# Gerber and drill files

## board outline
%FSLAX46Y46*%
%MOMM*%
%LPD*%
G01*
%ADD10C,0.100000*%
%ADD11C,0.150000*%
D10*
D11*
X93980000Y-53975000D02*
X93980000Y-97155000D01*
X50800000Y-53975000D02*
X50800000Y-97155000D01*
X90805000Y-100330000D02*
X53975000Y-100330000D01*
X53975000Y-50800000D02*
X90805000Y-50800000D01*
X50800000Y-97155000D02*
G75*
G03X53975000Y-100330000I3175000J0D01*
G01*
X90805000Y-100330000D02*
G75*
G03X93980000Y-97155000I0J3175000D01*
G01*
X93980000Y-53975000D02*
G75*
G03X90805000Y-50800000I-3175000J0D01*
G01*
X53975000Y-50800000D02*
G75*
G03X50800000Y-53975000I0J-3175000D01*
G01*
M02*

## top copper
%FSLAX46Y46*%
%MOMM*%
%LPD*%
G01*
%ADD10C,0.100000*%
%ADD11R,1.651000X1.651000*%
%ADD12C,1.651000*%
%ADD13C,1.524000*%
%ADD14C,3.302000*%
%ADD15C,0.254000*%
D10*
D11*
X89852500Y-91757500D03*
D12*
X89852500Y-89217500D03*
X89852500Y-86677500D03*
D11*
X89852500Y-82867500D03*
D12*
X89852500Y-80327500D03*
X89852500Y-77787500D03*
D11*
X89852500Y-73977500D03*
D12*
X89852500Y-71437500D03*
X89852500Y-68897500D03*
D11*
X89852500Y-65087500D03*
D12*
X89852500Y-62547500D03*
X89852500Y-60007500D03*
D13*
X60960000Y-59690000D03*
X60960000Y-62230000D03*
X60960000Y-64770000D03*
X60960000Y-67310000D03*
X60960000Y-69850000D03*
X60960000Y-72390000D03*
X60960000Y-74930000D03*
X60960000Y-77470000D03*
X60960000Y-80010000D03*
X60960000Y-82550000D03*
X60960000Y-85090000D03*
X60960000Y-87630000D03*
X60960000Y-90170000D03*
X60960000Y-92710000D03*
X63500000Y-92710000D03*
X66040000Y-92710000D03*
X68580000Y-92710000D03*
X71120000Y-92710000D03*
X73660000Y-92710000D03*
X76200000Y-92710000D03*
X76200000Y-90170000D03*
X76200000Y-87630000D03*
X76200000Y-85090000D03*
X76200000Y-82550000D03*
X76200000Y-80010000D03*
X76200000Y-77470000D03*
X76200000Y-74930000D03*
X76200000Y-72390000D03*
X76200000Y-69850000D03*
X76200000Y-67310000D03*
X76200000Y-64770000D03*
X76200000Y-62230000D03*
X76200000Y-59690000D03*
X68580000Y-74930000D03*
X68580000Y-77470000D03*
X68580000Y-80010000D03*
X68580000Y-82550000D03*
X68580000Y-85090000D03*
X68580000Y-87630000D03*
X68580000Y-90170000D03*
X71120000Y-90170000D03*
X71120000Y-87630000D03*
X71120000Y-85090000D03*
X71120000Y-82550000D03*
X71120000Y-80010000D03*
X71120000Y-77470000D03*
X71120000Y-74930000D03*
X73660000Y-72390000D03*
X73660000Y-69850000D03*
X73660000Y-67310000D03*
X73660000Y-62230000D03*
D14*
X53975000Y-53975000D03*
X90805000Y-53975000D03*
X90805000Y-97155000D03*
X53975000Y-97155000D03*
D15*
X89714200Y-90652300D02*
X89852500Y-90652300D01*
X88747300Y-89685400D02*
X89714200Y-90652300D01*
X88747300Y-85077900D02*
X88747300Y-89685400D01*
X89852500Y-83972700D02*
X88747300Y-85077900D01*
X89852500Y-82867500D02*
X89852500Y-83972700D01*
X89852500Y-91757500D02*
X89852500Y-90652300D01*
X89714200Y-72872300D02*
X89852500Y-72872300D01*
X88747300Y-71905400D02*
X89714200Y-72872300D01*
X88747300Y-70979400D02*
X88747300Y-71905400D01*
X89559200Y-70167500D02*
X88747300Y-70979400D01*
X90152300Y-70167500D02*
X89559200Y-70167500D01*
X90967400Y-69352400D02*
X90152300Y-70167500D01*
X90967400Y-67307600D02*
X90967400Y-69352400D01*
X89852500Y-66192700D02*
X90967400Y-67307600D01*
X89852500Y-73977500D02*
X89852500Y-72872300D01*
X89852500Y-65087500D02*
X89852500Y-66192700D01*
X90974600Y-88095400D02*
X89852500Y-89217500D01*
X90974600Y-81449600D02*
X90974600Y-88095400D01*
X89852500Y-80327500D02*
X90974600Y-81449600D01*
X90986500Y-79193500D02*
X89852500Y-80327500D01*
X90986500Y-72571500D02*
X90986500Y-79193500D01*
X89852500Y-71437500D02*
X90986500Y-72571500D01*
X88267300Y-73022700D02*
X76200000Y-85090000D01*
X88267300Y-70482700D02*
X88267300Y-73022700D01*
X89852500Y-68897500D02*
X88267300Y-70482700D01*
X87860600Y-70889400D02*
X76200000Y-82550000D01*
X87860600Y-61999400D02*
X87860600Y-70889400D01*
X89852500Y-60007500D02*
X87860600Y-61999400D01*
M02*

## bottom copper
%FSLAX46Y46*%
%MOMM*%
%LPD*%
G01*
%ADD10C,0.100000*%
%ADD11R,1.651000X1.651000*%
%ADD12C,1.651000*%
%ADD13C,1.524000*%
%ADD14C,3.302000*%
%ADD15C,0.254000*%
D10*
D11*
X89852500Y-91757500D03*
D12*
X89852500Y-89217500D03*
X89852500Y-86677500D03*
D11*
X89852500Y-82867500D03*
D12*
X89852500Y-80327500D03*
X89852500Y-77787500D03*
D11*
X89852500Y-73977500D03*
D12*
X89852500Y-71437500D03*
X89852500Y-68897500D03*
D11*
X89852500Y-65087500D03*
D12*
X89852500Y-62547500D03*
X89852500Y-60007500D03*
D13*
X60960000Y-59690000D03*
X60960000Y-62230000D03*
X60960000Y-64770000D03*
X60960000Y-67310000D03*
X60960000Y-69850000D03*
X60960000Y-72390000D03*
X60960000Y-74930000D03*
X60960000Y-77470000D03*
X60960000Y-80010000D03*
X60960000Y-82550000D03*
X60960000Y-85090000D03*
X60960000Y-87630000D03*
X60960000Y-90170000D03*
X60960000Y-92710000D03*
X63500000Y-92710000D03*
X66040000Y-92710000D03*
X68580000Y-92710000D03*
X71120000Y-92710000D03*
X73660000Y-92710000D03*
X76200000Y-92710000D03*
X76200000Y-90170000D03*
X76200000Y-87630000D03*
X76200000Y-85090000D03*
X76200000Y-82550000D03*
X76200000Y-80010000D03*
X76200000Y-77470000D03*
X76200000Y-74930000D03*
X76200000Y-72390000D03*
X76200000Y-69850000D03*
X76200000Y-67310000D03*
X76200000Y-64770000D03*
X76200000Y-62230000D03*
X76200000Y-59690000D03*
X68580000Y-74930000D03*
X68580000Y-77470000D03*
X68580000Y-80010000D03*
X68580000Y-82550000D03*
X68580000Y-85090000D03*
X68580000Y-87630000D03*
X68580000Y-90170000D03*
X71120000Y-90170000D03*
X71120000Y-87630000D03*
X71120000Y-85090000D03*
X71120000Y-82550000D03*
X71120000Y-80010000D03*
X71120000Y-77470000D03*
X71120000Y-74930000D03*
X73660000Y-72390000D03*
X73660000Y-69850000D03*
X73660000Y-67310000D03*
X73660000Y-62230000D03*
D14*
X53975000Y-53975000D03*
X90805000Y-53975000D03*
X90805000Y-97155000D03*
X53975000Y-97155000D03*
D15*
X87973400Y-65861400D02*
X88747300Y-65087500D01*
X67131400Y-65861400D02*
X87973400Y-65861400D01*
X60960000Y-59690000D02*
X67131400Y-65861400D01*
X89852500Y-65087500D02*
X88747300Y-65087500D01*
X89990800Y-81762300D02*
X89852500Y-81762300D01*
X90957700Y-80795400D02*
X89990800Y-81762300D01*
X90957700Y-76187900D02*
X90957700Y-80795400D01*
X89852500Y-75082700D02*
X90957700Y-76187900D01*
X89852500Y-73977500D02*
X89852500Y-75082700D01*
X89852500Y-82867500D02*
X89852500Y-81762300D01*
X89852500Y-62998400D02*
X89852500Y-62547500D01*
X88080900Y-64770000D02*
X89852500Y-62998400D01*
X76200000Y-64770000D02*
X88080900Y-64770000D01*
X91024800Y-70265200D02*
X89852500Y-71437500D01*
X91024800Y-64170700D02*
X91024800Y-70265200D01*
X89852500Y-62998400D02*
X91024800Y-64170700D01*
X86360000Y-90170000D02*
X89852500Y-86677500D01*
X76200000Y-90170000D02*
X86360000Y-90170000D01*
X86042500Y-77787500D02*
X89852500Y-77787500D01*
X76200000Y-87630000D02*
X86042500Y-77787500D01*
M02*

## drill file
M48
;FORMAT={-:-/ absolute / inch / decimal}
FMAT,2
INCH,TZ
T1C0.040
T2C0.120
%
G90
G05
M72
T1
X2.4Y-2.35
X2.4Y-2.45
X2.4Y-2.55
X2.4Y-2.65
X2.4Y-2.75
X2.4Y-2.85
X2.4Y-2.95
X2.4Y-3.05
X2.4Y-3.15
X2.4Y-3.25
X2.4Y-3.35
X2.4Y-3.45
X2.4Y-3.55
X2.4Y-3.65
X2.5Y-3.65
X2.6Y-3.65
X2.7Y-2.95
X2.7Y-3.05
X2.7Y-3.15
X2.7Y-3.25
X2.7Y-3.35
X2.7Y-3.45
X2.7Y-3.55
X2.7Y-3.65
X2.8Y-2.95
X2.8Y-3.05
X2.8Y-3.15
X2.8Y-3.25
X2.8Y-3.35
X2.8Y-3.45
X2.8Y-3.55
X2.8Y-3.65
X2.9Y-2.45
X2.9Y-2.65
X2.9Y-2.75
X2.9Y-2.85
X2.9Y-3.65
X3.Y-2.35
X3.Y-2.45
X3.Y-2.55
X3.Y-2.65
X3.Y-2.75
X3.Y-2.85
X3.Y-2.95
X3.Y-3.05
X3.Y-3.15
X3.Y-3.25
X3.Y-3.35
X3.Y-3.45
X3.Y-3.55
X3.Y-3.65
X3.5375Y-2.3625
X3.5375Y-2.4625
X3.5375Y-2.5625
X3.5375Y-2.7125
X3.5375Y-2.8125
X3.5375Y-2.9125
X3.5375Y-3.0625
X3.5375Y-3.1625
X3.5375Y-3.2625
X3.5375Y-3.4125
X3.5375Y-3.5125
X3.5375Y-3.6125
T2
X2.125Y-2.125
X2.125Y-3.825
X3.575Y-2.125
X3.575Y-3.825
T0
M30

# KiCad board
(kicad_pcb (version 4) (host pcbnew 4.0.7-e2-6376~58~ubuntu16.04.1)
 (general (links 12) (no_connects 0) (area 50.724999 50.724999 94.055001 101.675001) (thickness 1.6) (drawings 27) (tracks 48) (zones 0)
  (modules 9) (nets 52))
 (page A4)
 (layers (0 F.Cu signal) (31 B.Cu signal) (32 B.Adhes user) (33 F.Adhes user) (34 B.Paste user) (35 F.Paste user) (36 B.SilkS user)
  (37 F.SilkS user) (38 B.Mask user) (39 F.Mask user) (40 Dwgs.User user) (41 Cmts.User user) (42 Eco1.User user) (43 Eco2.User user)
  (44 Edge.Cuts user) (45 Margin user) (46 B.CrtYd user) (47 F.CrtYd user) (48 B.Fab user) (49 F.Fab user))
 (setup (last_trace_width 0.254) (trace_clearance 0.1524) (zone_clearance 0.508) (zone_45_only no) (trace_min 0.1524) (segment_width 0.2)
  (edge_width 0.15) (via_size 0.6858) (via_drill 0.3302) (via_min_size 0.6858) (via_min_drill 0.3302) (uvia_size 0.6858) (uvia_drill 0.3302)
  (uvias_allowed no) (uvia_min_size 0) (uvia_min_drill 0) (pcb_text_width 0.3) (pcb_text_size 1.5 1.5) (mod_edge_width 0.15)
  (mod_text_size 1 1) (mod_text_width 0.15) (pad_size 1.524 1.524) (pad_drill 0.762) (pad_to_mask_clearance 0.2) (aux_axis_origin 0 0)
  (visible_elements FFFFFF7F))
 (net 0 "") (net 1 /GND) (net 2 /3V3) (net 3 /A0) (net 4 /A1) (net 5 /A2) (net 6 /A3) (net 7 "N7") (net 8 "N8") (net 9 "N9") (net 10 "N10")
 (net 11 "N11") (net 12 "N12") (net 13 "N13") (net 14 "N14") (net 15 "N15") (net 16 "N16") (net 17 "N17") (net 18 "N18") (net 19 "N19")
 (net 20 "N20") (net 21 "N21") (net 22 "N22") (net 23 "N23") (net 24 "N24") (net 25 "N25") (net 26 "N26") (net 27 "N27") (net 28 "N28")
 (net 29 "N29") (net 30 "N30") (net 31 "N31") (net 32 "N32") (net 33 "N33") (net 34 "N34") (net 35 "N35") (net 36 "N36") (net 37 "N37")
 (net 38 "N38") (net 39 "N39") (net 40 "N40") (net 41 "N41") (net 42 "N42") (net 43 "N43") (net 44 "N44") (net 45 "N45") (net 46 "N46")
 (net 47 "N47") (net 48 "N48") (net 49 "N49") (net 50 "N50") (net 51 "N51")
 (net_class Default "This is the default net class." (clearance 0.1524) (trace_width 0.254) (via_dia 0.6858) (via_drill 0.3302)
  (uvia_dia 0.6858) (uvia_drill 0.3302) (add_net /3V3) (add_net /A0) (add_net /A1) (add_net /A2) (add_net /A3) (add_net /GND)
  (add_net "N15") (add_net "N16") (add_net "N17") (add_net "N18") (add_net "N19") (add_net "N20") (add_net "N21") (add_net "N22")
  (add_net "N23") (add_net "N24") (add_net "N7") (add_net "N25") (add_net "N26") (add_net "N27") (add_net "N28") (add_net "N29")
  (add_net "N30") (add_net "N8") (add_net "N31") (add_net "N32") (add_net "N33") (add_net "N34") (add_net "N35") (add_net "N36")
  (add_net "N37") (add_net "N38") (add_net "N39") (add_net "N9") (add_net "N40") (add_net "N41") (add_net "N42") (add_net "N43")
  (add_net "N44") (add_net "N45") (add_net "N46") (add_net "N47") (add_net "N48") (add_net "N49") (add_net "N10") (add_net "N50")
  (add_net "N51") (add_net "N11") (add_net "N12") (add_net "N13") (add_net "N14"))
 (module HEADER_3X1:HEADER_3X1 (layer F.Cu) (at 89.8525 89.2175 90)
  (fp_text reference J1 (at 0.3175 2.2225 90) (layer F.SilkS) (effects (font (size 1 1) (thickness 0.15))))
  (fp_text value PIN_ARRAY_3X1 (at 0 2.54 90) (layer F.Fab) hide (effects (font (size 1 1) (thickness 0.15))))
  (pad 1 thru_hole rect (at -2.54 0 90) (size 1.651 1.651) (drill 1.016) (layers *.Cu *.Mask) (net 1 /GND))
  (pad 2 thru_hole circle (at 0 0 90) (size 1.651 1.651) (drill 1.016) (layers *.Cu *.Mask) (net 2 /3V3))
  (pad 3 thru_hole circle (at 2.54 0 90) (size 1.651 1.651) (drill 1.016) (layers *.Cu *.Mask) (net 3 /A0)))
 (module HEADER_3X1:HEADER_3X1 (layer F.Cu) (at 89.8525 80.3275 90)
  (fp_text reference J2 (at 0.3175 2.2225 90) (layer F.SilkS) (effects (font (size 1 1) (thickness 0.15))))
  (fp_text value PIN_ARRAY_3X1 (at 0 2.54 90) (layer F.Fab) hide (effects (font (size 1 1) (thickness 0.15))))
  (pad 1 thru_hole rect (at -2.54 0 90) (size 1.651 1.651) (drill 1.016) (layers *.Cu *.Mask) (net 1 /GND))
  (pad 2 thru_hole circle (at 0 0 90) (size 1.651 1.651) (drill 1.016) (layers *.Cu *.Mask) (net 2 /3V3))
  (pad 3 thru_hole circle (at 2.54 0 90) (size 1.651 1.651) (drill 1.016) (layers *.Cu *.Mask) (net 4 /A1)))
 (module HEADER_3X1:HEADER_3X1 (layer F.Cu) (at 89.8525 71.4375 90)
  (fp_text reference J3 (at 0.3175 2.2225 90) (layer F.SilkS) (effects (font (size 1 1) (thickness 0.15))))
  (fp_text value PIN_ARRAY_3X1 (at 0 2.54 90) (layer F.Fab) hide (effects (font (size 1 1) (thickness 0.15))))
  (pad 1 thru_hole rect (at -2.54 0 90) (size 1.651 1.651) (drill 1.016) (layers *.Cu *.Mask) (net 1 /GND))
  (pad 2 thru_hole circle (at 0 0 90) (size 1.651 1.651) (drill 1.016) (layers *.Cu *.Mask) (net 2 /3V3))
  (pad 3 thru_hole circle (at 2.54 0 90) (size 1.651 1.651) (drill 1.016) (layers *.Cu *.Mask) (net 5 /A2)))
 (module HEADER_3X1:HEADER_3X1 (layer F.Cu) (at 89.8525 62.5475 90)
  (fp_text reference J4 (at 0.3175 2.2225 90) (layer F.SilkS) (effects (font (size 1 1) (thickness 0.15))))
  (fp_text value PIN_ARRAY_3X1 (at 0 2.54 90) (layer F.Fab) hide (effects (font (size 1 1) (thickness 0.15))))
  (pad 1 thru_hole rect (at -2.54 0 90) (size 1.651 1.651) (drill 1.016) (layers *.Cu *.Mask) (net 1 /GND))
  (pad 2 thru_hole circle (at 0 0 90) (size 1.651 1.651) (drill 1.016) (layers *.Cu *.Mask) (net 2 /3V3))
  (pad 3 thru_hole circle (at 2.54 0 90) (size 1.651 1.651) (drill 1.016) (layers *.Cu *.Mask) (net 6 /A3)))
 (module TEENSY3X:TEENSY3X (layer F.Cu) (at 68.58 76.2)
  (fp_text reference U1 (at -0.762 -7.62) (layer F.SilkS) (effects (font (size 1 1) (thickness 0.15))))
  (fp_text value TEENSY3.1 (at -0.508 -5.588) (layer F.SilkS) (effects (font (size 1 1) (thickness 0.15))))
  (pad 1 thru_hole circle (at -7.62 -16.51) (size 1.524 1.524) (drill 1.016) (layers *.Cu *.Mask F.SilkS) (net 1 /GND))
  (pad 2 thru_hole circle (at -7.62 -13.97) (size 1.524 1.524) (drill 1.016) (layers *.Cu *.Mask F.SilkS) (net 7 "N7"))
  (pad 3 thru_hole circle (at -7.62 -11.43) (size 1.524 1.524) (drill 1.016) (layers *.Cu *.Mask F.SilkS) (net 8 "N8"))
  (pad 4 thru_hole circle (at -7.62 -8.89) (size 1.524 1.524) (drill 1.016) (layers *.Cu *.Mask F.SilkS) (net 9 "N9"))
  (pad 5 thru_hole circle (at -7.62 -6.35) (size 1.524 1.524) (drill 1.016) (layers *.Cu *.Mask F.SilkS) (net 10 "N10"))
  (pad 6 thru_hole circle (at -7.62 -3.81) (size 1.524 1.524) (drill 1.016) (layers *.Cu *.Mask F.SilkS) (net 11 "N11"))
  (pad 7 thru_hole circle (at -7.62 -1.27) (size 1.524 1.524) (drill 1.016) (layers *.Cu *.Mask F.SilkS) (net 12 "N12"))
  (pad 8 thru_hole circle (at -7.62 1.27) (size 1.524 1.524) (drill 1.016) (layers *.Cu *.Mask F.SilkS) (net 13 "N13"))
  (pad 9 thru_hole circle (at -7.62 3.81) (size 1.524 1.524) (drill 1.016) (layers *.Cu *.Mask F.SilkS) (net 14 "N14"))
  (pad 10 thru_hole circle (at -7.62 6.35) (size 1.524 1.524) (drill 1.016) (layers *.Cu *.Mask F.SilkS) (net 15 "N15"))
  (pad 11 thru_hole circle (at -7.62 8.89) (size 1.524 1.524) (drill 1.016) (layers *.Cu *.Mask F.SilkS) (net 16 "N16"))
  (pad 12 thru_hole circle (at -7.62 11.43) (size 1.524 1.524) (drill 1.016) (layers *.Cu *.Mask F.SilkS) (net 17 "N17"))
  (pad 13 thru_hole circle (at -7.62 13.97) (size 1.524 1.524) (drill 1.016) (layers *.Cu *.Mask F.SilkS) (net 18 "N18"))
  (pad 14 thru_hole circle (at -7.62 16.51) (size 1.524 1.524) (drill 1.016) (layers *.Cu *.Mask F.SilkS) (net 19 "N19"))
  (pad 15 thru_hole circle (at -5.08 16.51) (size 1.524 1.524) (drill 1.016) (layers *.Cu *.Mask F.SilkS) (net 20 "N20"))
  (pad 16 thru_hole circle (at -2.54 16.51) (size 1.524 1.524) (drill 1.016) (layers *.Cu *.Mask F.SilkS) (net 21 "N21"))
  (pad 17 thru_hole circle (at 0 16.51) (size 1.524 1.524) (drill 1.016) (layers *.Cu *.Mask F.SilkS) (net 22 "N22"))
  (pad 18 thru_hole circle (at 2.54 16.51) (size 1.524 1.524) (drill 1.016) (layers *.Cu *.Mask F.SilkS) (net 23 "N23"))
  (pad 19 thru_hole circle (at 5.08 16.51) (size 1.524 1.524) (drill 1.016) (layers *.Cu *.Mask F.SilkS) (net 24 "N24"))
  (pad 20 thru_hole circle (at 7.62 16.51) (size 1.524 1.524) (drill 1.016) (layers *.Cu *.Mask F.SilkS) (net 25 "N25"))
  (pad 21 thru_hole circle (at 7.62 13.97) (size 1.524 1.524) (drill 1.016) (layers *.Cu *.Mask F.SilkS) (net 3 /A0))
  (pad 22 thru_hole circle (at 7.62 11.43) (size 1.524 1.524) (drill 1.016) (layers *.Cu *.Mask F.SilkS) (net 4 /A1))
  (pad 23 thru_hole circle (at 7.62 8.89) (size 1.524 1.524) (drill 1.016) (layers *.Cu *.Mask F.SilkS) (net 5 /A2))
  (pad 24 thru_hole circle (at 7.62 6.35) (size 1.524 1.524) (drill 1.016) (layers *.Cu *.Mask F.SilkS) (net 6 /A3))
  (pad 25 thru_hole circle (at 7.62 3.81) (size 1.524 1.524) (drill 1.016) (layers *.Cu *.Mask F.SilkS) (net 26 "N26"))
  (pad 26 thru_hole circle (at 7.62 1.27) (size 1.524 1.524) (drill 1.016) (layers *.Cu *.Mask F.SilkS) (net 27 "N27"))
  (pad 27 thru_hole circle (at 7.62 -1.27) (size 1.524 1.524) (drill 1.016) (layers *.Cu *.Mask F.SilkS) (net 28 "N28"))
  (pad 28 thru_hole circle (at 7.62 -3.81) (size 1.524 1.524) (drill 1.016) (layers *.Cu *.Mask F.SilkS) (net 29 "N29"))
  (pad 29 thru_hole circle (at 7.62 -6.35) (size 1.524 1.524) (drill 1.016) (layers *.Cu *.Mask F.SilkS) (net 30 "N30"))
  (pad 30 thru_hole circle (at 7.62 -8.89) (size 1.524 1.524) (drill 1.016) (layers *.Cu *.Mask F.SilkS) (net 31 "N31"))
  (pad 31 thru_hole circle (at 7.62 -11.43) (size 1.524 1.524) (drill 1.016) (layers *.Cu *.Mask F.SilkS) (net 2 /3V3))
  (pad 32 thru_hole circle (at 7.62 -13.97) (size 1.524 1.524) (drill 1.016) (layers *.Cu *.Mask F.SilkS) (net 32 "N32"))
  (pad 33 thru_hole circle (at 7.62 -16.51) (size 1.524 1.524) (drill 1.016) (layers *.Cu *.Mask F.SilkS) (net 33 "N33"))
  (pad 34 thru_hole circle (at 0 -1.27) (size 1.524 1.524) (drill 1.016) (layers *.Cu *.Mask F.SilkS) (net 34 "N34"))
  (pad 35 thru_hole circle (at 0 1.27) (size 1.524 1.524) (drill 1.016) (layers *.Cu *.Mask F.SilkS) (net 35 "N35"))
  (pad 36 thru_hole circle (at 0 3.81) (size 1.524 1.524) (drill 1.016) (layers *.Cu *.Mask F.SilkS) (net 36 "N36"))
  (pad 37 thru_hole circle (at 0 6.35) (size 1.524 1.524) (drill 1.016) (layers *.Cu *.Mask F.SilkS) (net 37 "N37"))
  (pad 38 thru_hole circle (at 0 8.89) (size 1.524 1.524) (drill 1.016) (layers *.Cu *.Mask F.SilkS) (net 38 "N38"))
  (pad 39 thru_hole circle (at 0 11.43) (size 1.524 1.524) (drill 1.016) (layers *.Cu *.Mask F.SilkS) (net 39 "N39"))
  (pad 40 thru_hole circle (at 0 13.97) (size 1.524 1.524) (drill 1.016) (layers *.Cu *.Mask F.SilkS) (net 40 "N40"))
  (pad 41 thru_hole circle (at 2.54 13.97) (size 1.524 1.524) (drill 1.016) (layers *.Cu *.Mask F.SilkS) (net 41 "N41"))
  (pad 42 thru_hole circle (at 2.54 11.43) (size 1.524 1.524) (drill 1.016) (layers *.Cu *.Mask F.SilkS) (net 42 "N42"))
  (pad 43 thru_hole circle (at 2.54 8.89) (size 1.524 1.524) (drill 1.016) (layers *.Cu *.Mask F.SilkS) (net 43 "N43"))
  (pad 44 thru_hole circle (at 2.54 6.35) (size 1.524 1.524) (drill 1.016) (layers *.Cu *.Mask F.SilkS) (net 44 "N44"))
  (pad 45 thru_hole circle (at 2.54 3.81) (size 1.524 1.524) (drill 1.016) (layers *.Cu *.Mask F.SilkS) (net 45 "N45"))
  (pad 46 thru_hole circle (at 2.54 1.27) (size 1.524 1.524) (drill 1.016) (layers *.Cu *.Mask F.SilkS) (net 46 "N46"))
  (pad 47 thru_hole circle (at 2.54 -1.27) (size 1.524 1.524) (drill 1.016) (layers *.Cu *.Mask F.SilkS) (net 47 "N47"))
  (pad 48 thru_hole circle (at 5.08 -3.81) (size 1.524 1.524) (drill 1.016) (layers *.Cu *.Mask F.SilkS) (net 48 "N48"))
  (pad 49 thru_hole circle (at 5.08 -6.35) (size 1.524 1.524) (drill 1.016) (layers *.Cu *.Mask F.SilkS) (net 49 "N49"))
  (pad 50 thru_hole circle (at 5.08 -8.89) (size 1.524 1.524) (drill 1.016) (layers *.Cu *.Mask F.SilkS) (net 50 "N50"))
  (pad 51 thru_hole circle (at 5.08 -13.97) (size 1.524 1.524) (drill 1.016) (layers *.Cu *.Mask F.SilkS) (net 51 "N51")))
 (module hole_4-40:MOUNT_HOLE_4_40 (layer F.Cu) (at 53.975 53.975)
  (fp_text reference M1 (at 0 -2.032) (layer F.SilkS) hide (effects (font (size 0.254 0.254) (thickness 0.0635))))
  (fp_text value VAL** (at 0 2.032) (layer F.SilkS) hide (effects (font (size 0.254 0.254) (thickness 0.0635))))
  (pad "" thru_hole circle (at 0 0) (size 3.302 3.302) (drill 3.048) (layers *.Cu *.SilkS *.Mask)))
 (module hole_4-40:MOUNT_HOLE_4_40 (layer F.Cu) (at 90.805 53.975)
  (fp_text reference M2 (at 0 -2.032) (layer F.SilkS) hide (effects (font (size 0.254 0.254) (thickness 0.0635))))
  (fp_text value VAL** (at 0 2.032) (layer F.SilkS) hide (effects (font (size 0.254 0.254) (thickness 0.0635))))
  (pad "" thru_hole circle (at 0 0) (size 3.302 3.302) (drill 3.048) (layers *.Cu *.SilkS *.Mask)))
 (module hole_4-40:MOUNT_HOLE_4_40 (layer F.Cu) (at 90.805 97.155)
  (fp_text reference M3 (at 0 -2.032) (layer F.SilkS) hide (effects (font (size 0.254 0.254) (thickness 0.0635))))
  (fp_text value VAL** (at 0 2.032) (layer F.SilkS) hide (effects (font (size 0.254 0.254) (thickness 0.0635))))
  (pad "" thru_hole circle (at 0 0) (size 3.302 3.302) (drill 3.048) (layers *.Cu *.SilkS *.Mask)))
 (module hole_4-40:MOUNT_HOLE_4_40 (layer F.Cu) (at 53.975 97.155)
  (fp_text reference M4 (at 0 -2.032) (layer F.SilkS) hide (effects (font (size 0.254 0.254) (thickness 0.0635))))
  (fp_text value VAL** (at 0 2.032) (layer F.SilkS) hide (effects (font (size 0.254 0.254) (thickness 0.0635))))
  (pad "" thru_hole circle (at 0 0) (size 3.302 3.302) (drill 3.048) (layers *.Cu *.SilkS *.Mask)))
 (gr_line (start 93.98 53.975) (end 93.98 97.155) (angle 90) (layer Edge.Cuts) (width 0.15))
 (gr_line (start 50.8 53.975) (end 50.8 97.155) (angle 90) (layer Edge.Cuts) (width 0.15))
 (gr_line (start 90.805 100.33) (end 53.975 100.33) (angle 90) (layer Edge.Cuts) (width 0.15))
 (gr_line (start 53.975 50.8) (end 90.805 50.8) (angle 90) (layer Edge.Cuts) (width 0.15))
 (gr_arc (start 53.975 97.155) (end 53.975 100.33) (angle 90) (layer Edge.Cuts) (width 0.15))
 (gr_arc (start 90.805 97.155) (end 93.98 97.155) (angle 90) (layer Edge.Cuts) (width 0.15))
 (gr_arc (start 90.805 53.975) (end 90.805 50.8) (angle 90) (layer Edge.Cuts) (width 0.15))
 (gr_arc (start 53.975 53.975) (end 50.8 53.975) (angle 90) (layer Edge.Cuts) (width 0.15))
 (segment (start 89.7142 90.6523) (end 89.8525 90.6523) (width 0.254) (layer F.Cu) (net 1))
 (segment (start 88.7473 89.6854) (end 89.7142 90.6523) (width 0.254) (layer F.Cu) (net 1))
 (segment (start 88.7473 85.0779) (end 88.7473 89.6854) (width 0.254) (layer F.Cu) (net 1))
 (segment (start 89.8525 83.9727) (end 88.7473 85.0779) (width 0.254) (layer F.Cu) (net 1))
 (segment (start 89.8525 82.8675) (end 89.8525 83.9727) (width 0.254) (layer F.Cu) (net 1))
 (segment (start 89.8525 91.7575) (end 89.8525 90.6523) (width 0.254) (layer F.Cu) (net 1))
 (segment (start 87.9734 65.8614) (end 88.7473 65.0875) (width 0.254) (layer B.Cu) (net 1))
 (segment (start 67.1314 65.8614) (end 87.9734 65.8614) (width 0.254) (layer B.Cu) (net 1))
 (segment (start 60.96 59.69) (end 67.1314 65.8614) (width 0.254) (layer B.Cu) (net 1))
 (segment (start 89.8525 65.0875) (end 88.7473 65.0875) (width 0.254) (layer B.Cu) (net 1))
 (segment (start 89.7142 72.8723) (end 89.8525 72.8723) (width 0.254) (layer F.Cu) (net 1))
 (segment (start 88.7473 71.9054) (end 89.7142 72.8723) (width 0.254) (layer F.Cu) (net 1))
 (segment (start 88.7473 70.9794) (end 88.7473 71.9054) (width 0.254) (layer F.Cu) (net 1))
 (segment (start 89.5592 70.1675) (end 88.7473 70.9794) (width 0.254) (layer F.Cu) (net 1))
 (segment (start 90.1523 70.1675) (end 89.5592 70.1675) (width 0.254) (layer F.Cu) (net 1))
 (segment (start 90.9674 69.3524) (end 90.1523 70.1675) (width 0.254) (layer F.Cu) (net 1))
 (segment (start 90.9674 67.3076) (end 90.9674 69.3524) (width 0.254) (layer F.Cu) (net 1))
 (segment (start 89.8525 66.1927) (end 90.9674 67.3076) (width 0.254) (layer F.Cu) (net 1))
 (segment (start 89.8525 73.9775) (end 89.8525 72.8723) (width 0.254) (layer F.Cu) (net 1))
 (segment (start 89.8525 65.0875) (end 89.8525 66.1927) (width 0.254) (layer F.Cu) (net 1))
 (segment (start 89.9908 81.7623) (end 89.8525 81.7623) (width 0.254) (layer B.Cu) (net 1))
 (segment (start 90.9577 80.7954) (end 89.9908 81.7623) (width 0.254) (layer B.Cu) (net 1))
 (segment (start 90.9577 76.1879) (end 90.9577 80.7954) (width 0.254) (layer B.Cu) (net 1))
 (segment (start 89.8525 75.0827) (end 90.9577 76.1879) (width 0.254) (layer B.Cu) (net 1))
 (segment (start 89.8525 73.9775) (end 89.8525 75.0827) (width 0.254) (layer B.Cu) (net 1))
 (segment (start 89.8525 82.8675) (end 89.8525 81.7623) (width 0.254) (layer B.Cu) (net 1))
 (segment (start 90.9746 88.0954) (end 89.8525 89.2175) (width 0.254) (layer F.Cu) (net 2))
 (segment (start 90.9746 81.4496) (end 90.9746 88.0954) (width 0.254) (layer F.Cu) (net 2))
 (segment (start 89.8525 80.3275) (end 90.9746 81.4496) (width 0.254) (layer F.Cu) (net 2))
 (segment (start 90.9865 79.1935) (end 89.8525 80.3275) (width 0.254) (layer F.Cu) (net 2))
 (segment (start 90.9865 72.5715) (end 90.9865 79.1935) (width 0.254) (layer F.Cu) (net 2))
 (segment (start 89.8525 71.4375) (end 90.9865 72.5715) (width 0.254) (layer F.Cu) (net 2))
 (segment (start 89.8525 62.9984) (end 89.8525 62.5475) (width 0.254) (layer B.Cu) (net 2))
 (segment (start 88.0809 64.77) (end 89.8525 62.9984) (width 0.254) (layer B.Cu) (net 2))
 (segment (start 76.2 64.77) (end 88.0809 64.77) (width 0.254) (layer B.Cu) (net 2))
 (segment (start 91.0248 70.2652) (end 89.8525 71.4375) (width 0.254) (layer B.Cu) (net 2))
 (segment (start 91.0248 64.1707) (end 91.0248 70.2652) (width 0.254) (layer B.Cu) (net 2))
 (segment (start 89.8525 62.9984) (end 91.0248 64.1707) (width 0.254) (layer B.Cu) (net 2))
 (segment (start 86.36 90.17) (end 89.8525 86.6775) (width 0.254) (layer B.Cu) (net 3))
 (segment (start 76.2 90.17) (end 86.36 90.17) (width 0.254) (layer B.Cu) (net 3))
 (segment (start 86.0425 77.7875) (end 89.8525 77.7875) (width 0.254) (layer B.Cu) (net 4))
 (segment (start 76.2 87.63) (end 86.0425 77.7875) (width 0.254) (layer B.Cu) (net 4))
 (segment (start 88.2673 73.0227) (end 76.2 85.09) (width 0.254) (layer F.Cu) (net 5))
 (segment (start 88.2673 70.4827) (end 88.2673 73.0227) (width 0.254) (layer F.Cu) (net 5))
 (segment (start 89.8525 68.8975) (end 88.2673 70.4827) (width 0.254) (layer F.Cu) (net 5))
 (segment (start 87.8606 70.8894) (end 76.2 82.55) (width 0.254) (layer F.Cu) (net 6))
 (segment (start 87.8606 61.9994) (end 87.8606 70.8894) (width 0.254) (layer F.Cu) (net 6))
 (segment (start 89.8525 60.0075) (end 87.8606 61.9994) (width 0.254) (layer F.Cu) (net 6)))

